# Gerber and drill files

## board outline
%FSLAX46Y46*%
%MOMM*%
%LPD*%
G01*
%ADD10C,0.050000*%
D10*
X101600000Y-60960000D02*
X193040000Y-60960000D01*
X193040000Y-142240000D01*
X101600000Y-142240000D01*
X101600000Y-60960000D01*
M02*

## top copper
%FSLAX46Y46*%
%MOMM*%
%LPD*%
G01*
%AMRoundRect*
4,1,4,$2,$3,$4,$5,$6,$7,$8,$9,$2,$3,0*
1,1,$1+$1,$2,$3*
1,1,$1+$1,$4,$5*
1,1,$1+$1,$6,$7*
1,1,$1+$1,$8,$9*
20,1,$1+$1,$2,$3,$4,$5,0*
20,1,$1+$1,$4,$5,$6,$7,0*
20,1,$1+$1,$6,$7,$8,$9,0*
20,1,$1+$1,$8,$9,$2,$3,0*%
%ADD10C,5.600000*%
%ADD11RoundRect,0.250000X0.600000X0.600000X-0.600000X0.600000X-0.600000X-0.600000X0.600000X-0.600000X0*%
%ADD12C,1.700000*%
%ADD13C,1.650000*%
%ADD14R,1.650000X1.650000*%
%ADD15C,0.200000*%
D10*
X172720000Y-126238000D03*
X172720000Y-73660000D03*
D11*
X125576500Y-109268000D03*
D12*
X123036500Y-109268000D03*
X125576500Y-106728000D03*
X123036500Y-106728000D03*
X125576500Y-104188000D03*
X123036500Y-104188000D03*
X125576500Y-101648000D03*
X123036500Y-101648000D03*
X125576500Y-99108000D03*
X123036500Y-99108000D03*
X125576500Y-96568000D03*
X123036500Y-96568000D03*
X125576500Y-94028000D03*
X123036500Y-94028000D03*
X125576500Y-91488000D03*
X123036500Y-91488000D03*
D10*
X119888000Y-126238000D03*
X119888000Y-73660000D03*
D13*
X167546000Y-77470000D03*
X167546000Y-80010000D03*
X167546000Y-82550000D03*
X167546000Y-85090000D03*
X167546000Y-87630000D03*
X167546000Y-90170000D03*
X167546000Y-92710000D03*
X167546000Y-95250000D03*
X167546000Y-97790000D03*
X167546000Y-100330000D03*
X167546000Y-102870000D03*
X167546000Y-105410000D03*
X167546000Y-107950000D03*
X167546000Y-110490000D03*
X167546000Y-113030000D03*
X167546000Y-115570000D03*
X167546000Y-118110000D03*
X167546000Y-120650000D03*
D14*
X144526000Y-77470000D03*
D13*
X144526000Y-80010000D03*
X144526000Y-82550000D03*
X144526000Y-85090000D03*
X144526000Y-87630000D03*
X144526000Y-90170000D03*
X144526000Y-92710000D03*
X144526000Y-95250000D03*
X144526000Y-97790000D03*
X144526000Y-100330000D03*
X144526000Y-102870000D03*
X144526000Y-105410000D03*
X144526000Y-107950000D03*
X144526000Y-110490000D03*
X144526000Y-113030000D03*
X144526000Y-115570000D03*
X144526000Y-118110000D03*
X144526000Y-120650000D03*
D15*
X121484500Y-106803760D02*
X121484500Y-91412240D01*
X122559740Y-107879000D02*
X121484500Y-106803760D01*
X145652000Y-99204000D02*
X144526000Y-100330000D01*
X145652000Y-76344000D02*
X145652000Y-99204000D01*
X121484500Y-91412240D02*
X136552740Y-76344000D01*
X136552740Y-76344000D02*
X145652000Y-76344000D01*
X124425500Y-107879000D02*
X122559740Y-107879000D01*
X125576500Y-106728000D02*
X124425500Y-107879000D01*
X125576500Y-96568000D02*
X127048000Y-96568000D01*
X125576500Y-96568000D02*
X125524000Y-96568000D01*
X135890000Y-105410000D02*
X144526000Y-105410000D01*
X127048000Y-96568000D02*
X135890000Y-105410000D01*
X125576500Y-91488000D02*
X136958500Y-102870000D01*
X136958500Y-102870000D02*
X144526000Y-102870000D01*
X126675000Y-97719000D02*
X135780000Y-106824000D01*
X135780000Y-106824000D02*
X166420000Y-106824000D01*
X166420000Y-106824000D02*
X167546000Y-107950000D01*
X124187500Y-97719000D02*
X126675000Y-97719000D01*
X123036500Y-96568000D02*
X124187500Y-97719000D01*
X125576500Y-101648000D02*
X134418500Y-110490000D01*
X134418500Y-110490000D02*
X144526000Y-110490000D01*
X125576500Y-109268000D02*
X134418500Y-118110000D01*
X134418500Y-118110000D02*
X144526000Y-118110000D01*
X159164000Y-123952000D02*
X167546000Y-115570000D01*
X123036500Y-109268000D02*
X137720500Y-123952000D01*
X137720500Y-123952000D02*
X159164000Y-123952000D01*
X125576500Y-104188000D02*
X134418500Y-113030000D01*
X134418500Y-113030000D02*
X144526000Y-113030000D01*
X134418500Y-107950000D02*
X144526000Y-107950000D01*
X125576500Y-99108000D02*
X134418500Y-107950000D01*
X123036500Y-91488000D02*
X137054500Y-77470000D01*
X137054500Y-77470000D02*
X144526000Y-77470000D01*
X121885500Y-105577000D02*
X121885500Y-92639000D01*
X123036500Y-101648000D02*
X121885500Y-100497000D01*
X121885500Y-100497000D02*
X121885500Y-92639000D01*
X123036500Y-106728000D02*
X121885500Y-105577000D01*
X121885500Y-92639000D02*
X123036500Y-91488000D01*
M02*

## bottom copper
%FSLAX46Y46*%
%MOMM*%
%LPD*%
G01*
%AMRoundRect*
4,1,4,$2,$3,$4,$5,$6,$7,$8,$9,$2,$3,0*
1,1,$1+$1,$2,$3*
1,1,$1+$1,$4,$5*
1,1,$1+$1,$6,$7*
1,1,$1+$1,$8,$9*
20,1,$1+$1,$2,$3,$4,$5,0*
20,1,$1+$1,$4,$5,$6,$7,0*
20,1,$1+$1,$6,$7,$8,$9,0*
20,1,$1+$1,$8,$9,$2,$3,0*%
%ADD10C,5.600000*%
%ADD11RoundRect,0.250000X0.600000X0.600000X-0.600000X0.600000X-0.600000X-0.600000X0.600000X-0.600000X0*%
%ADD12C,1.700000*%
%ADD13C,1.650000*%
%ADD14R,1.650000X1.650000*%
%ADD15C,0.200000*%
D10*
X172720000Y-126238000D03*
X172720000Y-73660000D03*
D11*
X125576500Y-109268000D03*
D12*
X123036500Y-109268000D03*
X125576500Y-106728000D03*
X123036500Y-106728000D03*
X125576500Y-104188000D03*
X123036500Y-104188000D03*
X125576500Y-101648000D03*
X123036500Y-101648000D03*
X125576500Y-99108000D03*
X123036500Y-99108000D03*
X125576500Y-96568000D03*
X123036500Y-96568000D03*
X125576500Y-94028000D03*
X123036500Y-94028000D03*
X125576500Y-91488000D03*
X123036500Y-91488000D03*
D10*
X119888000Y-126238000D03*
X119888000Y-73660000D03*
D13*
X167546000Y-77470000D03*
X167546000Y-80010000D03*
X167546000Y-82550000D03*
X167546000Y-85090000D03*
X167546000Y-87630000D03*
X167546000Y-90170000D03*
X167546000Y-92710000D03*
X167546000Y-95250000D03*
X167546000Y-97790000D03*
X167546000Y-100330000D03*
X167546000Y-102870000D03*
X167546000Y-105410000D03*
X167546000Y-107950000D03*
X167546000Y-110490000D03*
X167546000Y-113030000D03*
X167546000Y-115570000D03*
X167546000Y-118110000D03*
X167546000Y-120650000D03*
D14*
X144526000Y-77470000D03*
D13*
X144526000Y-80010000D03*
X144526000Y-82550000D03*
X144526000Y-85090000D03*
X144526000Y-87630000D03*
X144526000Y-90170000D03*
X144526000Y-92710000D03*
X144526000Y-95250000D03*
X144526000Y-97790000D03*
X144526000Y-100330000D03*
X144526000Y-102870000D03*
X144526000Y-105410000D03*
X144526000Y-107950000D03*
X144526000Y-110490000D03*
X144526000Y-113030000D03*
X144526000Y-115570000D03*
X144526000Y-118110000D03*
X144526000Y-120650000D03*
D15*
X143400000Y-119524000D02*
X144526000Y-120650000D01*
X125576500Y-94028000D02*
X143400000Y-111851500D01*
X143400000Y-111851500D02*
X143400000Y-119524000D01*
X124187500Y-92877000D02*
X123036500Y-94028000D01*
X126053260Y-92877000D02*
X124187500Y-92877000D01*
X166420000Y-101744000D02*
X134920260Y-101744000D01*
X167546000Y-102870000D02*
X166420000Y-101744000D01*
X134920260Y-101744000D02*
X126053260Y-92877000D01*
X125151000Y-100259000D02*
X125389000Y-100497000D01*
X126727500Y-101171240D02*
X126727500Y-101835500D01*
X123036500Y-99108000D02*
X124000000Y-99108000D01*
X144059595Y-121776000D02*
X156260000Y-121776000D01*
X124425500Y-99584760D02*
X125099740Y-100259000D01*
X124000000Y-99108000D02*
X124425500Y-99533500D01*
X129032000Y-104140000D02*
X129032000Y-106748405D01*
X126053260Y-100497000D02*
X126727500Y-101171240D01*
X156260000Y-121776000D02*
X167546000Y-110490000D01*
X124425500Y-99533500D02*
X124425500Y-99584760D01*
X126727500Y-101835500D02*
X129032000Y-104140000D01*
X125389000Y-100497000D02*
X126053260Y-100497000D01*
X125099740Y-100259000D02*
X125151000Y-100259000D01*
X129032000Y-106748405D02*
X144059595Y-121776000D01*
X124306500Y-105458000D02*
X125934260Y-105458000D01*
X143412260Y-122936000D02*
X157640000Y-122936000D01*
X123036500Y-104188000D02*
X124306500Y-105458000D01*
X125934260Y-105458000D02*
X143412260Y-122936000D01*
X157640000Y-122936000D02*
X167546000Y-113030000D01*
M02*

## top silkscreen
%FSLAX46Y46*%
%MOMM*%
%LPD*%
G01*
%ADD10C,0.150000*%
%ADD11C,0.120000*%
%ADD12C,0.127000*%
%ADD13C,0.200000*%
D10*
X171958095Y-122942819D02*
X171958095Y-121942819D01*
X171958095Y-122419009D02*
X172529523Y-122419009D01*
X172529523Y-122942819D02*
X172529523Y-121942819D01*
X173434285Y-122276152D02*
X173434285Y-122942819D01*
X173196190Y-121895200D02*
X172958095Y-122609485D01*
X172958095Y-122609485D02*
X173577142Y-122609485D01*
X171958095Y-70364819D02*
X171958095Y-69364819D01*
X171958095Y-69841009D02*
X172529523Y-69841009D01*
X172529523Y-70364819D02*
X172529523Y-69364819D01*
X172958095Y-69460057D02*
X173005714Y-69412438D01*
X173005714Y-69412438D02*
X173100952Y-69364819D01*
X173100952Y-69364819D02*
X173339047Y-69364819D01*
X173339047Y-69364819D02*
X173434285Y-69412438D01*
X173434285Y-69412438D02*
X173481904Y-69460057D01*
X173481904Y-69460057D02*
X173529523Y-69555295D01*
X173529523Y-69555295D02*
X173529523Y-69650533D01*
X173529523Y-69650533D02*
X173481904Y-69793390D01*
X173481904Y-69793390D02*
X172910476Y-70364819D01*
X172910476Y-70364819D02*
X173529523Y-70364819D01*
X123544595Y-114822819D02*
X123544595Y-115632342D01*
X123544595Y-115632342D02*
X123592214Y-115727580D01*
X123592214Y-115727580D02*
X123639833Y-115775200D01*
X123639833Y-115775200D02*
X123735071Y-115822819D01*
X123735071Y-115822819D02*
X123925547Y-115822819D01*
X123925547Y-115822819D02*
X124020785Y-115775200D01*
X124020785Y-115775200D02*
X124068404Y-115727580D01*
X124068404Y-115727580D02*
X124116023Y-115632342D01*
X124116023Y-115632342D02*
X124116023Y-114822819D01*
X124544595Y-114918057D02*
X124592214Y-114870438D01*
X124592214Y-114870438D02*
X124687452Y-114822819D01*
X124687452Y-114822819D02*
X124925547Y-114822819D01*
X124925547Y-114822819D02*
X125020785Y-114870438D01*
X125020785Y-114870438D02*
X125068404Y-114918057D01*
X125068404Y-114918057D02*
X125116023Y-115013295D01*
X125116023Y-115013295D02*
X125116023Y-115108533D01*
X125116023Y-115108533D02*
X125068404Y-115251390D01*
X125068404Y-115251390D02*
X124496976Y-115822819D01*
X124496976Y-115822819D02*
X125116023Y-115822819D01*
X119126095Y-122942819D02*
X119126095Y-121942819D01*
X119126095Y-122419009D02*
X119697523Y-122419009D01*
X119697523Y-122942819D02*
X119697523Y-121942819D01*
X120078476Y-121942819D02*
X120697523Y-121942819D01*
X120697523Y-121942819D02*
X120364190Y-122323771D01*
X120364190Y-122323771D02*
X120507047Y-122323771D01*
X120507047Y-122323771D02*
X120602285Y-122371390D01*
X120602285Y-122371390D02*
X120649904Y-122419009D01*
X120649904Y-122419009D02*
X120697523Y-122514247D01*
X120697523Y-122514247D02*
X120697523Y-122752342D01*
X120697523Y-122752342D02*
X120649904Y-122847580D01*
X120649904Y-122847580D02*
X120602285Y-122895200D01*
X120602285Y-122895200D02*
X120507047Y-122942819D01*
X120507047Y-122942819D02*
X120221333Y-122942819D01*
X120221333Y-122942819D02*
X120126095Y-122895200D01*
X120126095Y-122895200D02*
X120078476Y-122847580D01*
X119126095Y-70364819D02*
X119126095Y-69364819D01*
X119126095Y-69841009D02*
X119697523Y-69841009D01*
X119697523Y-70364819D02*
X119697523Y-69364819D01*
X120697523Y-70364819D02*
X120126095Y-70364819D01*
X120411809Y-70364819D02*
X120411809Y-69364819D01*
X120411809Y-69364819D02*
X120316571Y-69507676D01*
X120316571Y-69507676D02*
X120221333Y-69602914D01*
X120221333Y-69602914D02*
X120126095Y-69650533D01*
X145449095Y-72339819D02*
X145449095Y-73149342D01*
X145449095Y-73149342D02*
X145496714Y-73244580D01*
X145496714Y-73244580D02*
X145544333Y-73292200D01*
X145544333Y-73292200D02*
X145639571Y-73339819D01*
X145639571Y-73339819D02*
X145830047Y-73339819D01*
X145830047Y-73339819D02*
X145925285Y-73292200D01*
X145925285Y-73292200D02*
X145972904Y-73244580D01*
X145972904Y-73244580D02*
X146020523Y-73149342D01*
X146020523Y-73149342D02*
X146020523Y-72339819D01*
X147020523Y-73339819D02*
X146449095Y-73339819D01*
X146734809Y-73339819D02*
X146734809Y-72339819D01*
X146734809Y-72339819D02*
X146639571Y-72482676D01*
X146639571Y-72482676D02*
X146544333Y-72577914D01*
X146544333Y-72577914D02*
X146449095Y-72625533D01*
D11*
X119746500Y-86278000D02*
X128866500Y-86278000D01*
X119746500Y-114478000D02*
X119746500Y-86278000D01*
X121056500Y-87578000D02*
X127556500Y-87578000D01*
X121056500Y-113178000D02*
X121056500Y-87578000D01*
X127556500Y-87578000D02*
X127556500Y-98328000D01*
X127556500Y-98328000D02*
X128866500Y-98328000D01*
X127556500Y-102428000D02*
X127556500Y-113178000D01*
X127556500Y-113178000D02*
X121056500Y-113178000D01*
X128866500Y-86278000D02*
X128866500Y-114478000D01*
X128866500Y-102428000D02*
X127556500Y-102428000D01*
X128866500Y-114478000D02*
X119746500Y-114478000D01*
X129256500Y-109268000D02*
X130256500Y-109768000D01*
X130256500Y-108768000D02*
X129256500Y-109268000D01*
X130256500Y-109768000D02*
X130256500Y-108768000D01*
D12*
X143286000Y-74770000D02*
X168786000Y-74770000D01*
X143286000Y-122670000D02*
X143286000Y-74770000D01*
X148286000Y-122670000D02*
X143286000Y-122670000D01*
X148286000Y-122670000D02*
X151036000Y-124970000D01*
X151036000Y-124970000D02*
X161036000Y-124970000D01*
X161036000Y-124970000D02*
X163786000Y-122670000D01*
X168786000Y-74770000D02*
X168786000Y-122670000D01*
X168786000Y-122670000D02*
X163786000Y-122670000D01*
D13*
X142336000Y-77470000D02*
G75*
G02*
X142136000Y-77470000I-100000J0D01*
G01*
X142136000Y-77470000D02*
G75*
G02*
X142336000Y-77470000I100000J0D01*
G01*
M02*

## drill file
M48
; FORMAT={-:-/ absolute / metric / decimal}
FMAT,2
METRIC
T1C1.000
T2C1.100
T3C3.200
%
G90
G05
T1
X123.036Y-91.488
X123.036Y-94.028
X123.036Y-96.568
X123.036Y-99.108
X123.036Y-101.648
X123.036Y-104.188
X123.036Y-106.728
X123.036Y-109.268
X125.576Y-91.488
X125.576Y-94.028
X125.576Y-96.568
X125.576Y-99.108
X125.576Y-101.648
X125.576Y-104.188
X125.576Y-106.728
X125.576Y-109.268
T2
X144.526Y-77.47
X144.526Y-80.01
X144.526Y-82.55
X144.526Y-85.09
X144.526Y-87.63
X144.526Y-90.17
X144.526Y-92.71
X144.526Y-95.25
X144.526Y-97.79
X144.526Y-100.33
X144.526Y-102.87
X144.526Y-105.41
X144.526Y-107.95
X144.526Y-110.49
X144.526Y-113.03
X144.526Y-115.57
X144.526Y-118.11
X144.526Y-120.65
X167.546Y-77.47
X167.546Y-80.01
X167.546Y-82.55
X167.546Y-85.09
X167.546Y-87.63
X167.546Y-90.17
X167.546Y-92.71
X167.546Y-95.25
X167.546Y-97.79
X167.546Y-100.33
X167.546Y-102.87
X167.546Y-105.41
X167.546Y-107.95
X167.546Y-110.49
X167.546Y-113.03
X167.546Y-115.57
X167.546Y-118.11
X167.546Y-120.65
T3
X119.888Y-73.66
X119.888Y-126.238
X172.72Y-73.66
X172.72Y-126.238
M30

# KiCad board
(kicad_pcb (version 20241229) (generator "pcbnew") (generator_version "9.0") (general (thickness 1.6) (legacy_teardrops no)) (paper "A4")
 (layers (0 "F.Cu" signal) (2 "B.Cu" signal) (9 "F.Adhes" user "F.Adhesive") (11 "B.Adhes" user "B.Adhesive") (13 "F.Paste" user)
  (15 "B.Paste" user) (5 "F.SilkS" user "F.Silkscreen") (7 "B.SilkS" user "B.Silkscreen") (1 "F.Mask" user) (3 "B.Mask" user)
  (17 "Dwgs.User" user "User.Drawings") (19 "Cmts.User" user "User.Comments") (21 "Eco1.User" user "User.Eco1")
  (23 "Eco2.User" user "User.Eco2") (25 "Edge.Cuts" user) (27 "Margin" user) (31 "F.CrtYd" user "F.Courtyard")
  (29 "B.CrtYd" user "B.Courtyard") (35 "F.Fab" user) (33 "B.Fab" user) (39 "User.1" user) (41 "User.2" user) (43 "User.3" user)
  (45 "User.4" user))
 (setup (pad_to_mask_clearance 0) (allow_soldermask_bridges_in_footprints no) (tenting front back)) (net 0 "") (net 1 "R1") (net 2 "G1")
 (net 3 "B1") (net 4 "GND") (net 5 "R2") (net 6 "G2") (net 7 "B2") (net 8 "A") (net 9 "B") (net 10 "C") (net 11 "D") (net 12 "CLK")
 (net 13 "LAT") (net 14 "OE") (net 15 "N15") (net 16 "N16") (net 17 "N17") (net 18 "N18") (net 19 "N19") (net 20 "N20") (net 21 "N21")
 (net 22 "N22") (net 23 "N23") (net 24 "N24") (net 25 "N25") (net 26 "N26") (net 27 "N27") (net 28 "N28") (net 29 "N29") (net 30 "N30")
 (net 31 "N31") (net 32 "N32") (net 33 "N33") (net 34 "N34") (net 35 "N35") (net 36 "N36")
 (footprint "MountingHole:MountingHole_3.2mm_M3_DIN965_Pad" (layer "F.Cu") (at 172.72 126.238)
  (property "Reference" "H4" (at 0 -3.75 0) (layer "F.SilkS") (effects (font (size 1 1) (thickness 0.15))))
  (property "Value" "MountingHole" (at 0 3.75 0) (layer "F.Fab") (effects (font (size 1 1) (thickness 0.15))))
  (pad "1" thru_hole circle (at 0 0) (size 5.6 5.6) (drill 3.2) (layers "*.Cu" "*.Mask") (remove_unused_layers no) (zone_connect 2)))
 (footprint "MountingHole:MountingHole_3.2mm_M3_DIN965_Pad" (layer "F.Cu") (at 172.72 73.66)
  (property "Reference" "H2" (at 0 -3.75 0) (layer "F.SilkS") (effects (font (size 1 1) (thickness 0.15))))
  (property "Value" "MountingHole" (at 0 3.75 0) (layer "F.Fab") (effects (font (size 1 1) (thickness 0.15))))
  (pad "1" thru_hole circle (at 0 0) (size 5.6 5.6) (drill 3.2) (layers "*.Cu" "*.Mask") (remove_unused_layers no) (zone_connect 2)))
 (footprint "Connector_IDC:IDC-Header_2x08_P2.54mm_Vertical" (layer "F.Cu") (at 125.5765 109.268 180)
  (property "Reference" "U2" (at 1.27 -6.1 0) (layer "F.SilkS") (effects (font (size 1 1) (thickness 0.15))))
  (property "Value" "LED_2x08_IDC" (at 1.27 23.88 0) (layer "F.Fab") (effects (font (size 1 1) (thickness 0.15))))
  (fp_line (start 5.83 22.99) (end -3.29 22.99) (stroke (width 0.12) (type solid)) (layer "F.SilkS"))
  (fp_line (start 5.83 -5.21) (end 5.83 22.99) (stroke (width 0.12) (type solid)) (layer "F.SilkS"))
  (fp_line (start 4.52 21.69) (end -1.98 21.69) (stroke (width 0.12) (type solid)) (layer "F.SilkS"))
  (fp_line (start 4.52 -3.91) (end 4.52 21.69) (stroke (width 0.12) (type solid)) (layer "F.SilkS"))
  (fp_line (start -1.98 21.69) (end -1.98 10.94) (stroke (width 0.12) (type solid)) (layer "F.SilkS"))
  (fp_line (start -1.98 10.94) (end -3.29 10.94) (stroke (width 0.12) (type solid)) (layer "F.SilkS"))
  (fp_line (start -1.98 6.84) (end -1.98 -3.91) (stroke (width 0.12) (type solid)) (layer "F.SilkS"))
  (fp_line (start -1.98 -3.91) (end 4.52 -3.91) (stroke (width 0.12) (type solid)) (layer "F.SilkS"))
  (fp_line (start -3.29 22.99) (end -3.29 -5.21) (stroke (width 0.12) (type solid)) (layer "F.SilkS"))
  (fp_line (start -3.29 6.84) (end -1.98 6.84) (stroke (width 0.12) (type solid)) (layer "F.SilkS"))
  (fp_line (start -3.29 -5.21) (end 5.83 -5.21) (stroke (width 0.12) (type solid)) (layer "F.SilkS"))
  (fp_line (start -3.68 0) (end -4.68 -0.5) (stroke (width 0.12) (type solid)) (layer "F.SilkS"))
  (fp_line (start -4.68 0.5) (end -3.68 0) (stroke (width 0.12) (type solid)) (layer "F.SilkS"))
  (fp_line (start -4.68 -0.5) (end -4.68 0.5) (stroke (width 0.12) (type solid)) (layer "F.SilkS"))
  (pad "1" thru_hole roundrect (at 0 0 180) (size 1.7 1.7) (drill 1) (layers "*.Cu" "*.Mask") (remove_unused_layers no)
   (roundrect_rratio 0.147059) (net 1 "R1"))
  (pad "2" thru_hole circle (at 2.54 0 180) (size 1.7 1.7) (drill 1) (layers "*.Cu" "*.Mask") (remove_unused_layers no) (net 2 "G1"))
  (pad "3" thru_hole circle (at 0 2.54 180) (size 1.7 1.7) (drill 1) (layers "*.Cu" "*.Mask") (remove_unused_layers no) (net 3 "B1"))
  (pad "4" thru_hole circle (at 2.54 2.54 180) (size 1.7 1.7) (drill 1) (layers "*.Cu" "*.Mask") (remove_unused_layers no) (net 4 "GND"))
  (pad "5" thru_hole circle (at 0 5.08 180) (size 1.7 1.7) (drill 1) (layers "*.Cu" "*.Mask") (remove_unused_layers no) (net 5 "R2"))
  (pad "6" thru_hole circle (at 2.54 5.08 180) (size 1.7 1.7) (drill 1) (layers "*.Cu" "*.Mask") (remove_unused_layers no) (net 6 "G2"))
  (pad "7" thru_hole circle (at 0 7.62 180) (size 1.7 1.7) (drill 1) (layers "*.Cu" "*.Mask") (remove_unused_layers no) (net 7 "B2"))
  (pad "8" thru_hole circle (at 2.54 7.62 180) (size 1.7 1.7) (drill 1) (layers "*.Cu" "*.Mask") (remove_unused_layers no) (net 4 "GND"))
  (pad "9" thru_hole circle (at 0 10.16 180) (size 1.7 1.7) (drill 1) (layers "*.Cu" "*.Mask") (remove_unused_layers no) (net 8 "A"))
  (pad "10" thru_hole circle (at 2.54 10.16 180) (size 1.7 1.7) (drill 1) (layers "*.Cu" "*.Mask") (remove_unused_layers no) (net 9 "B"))
  (pad "11" thru_hole circle (at 0 12.7 180) (size 1.7 1.7) (drill 1) (layers "*.Cu" "*.Mask") (remove_unused_layers no) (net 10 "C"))
  (pad "12" thru_hole circle (at 2.54 12.7 180) (size 1.7 1.7) (drill 1) (layers "*.Cu" "*.Mask") (remove_unused_layers no) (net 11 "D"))
  (pad "13" thru_hole circle (at 0 15.24 180) (size 1.7 1.7) (drill 1) (layers "*.Cu" "*.Mask") (remove_unused_layers no) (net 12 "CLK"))
  (pad "14" thru_hole circle (at 2.54 15.24 180) (size 1.7 1.7) (drill 1) (layers "*.Cu" "*.Mask") (remove_unused_layers no) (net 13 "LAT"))
  (pad "15" thru_hole circle (at 0 17.78 180) (size 1.7 1.7) (drill 1) (layers "*.Cu" "*.Mask") (remove_unused_layers no) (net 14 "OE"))
  (pad "16" thru_hole circle (at 2.54 17.78 180) (size 1.7 1.7) (drill 1) (layers "*.Cu" "*.Mask") (remove_unused_layers no) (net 4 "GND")))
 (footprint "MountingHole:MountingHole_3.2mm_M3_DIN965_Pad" (layer "F.Cu") (at 119.888 126.238)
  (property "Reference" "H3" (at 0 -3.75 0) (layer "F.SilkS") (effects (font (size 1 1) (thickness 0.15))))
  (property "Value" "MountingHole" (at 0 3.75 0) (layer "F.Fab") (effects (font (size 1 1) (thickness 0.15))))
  (pad "1" thru_hole circle (at 0 0) (size 5.6 5.6) (drill 3.2) (layers "*.Cu" "*.Mask") (remove_unused_layers no) (zone_connect 2)))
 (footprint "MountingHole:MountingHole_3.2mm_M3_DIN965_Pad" (layer "F.Cu") (at 119.888 73.66)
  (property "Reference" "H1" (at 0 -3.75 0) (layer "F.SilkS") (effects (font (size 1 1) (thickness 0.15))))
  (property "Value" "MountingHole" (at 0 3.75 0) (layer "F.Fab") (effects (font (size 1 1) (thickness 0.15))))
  (pad "1" thru_hole circle (at 0 0) (size 5.6 5.6) (drill 3.2) (layers "*.Cu" "*.Mask") (remove_unused_layers no) (zone_connect 2)))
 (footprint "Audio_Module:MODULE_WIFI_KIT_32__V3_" (layer "F.Cu") (at 156.036 99.87)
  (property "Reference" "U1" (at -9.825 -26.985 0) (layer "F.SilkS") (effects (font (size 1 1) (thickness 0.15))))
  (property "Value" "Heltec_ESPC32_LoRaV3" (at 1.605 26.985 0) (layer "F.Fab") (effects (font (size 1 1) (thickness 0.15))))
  (fp_line (start -12.75 -25.1) (end 12.75 -25.1) (stroke (width 0.127) (type solid)) (layer "F.SilkS"))
  (fp_line (start -12.75 22.8) (end -12.75 -25.1) (stroke (width 0.127) (type solid)) (layer "F.SilkS"))
  (fp_line (start -7.75 22.8) (end -12.75 22.8) (stroke (width 0.127) (type solid)) (layer "F.SilkS"))
  (fp_line (start -7.75 22.8) (end -5 25.1) (stroke (width 0.127) (type solid)) (layer "F.SilkS"))
  (fp_line (start -5 25.1) (end 5 25.1) (stroke (width 0.127) (type solid)) (layer "F.SilkS"))
  (fp_line (start 5 25.1) (end 7.75 22.8) (stroke (width 0.127) (type solid)) (layer "F.SilkS"))
  (fp_line (start 12.75 -25.1) (end 12.75 22.8) (stroke (width 0.127) (type solid)) (layer "F.SilkS"))
  (fp_line (start 12.75 22.8) (end 7.75 22.8) (stroke (width 0.127) (type solid)) (layer "F.SilkS"))
  (fp_circle (center -13.8 -22.4) (end -13.7 -22.4) (stroke (width 0.2) (type solid)) (fill no) (layer "F.SilkS"))
  (pad "1" thru_hole circle (at 11.51 -22.4) (size 1.65 1.65) (drill 1.1) (layers "*.Cu" "*.Mask") (remove_unused_layers no) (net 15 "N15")
   (solder_mask_margin 0.102))
  (pad "2" thru_hole circle (at 11.51 -19.86) (size 1.65 1.65) (drill 1.1) (layers "*.Cu" "*.Mask") (remove_unused_layers no) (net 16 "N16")
   (solder_mask_margin 0.102))
  (pad "3" thru_hole circle (at 11.51 -17.32) (size 1.65 1.65) (drill 1.1) (layers "*.Cu" "*.Mask") (remove_unused_layers no) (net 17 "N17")
   (solder_mask_margin 0.102))
  (pad "4" thru_hole circle (at 11.51 -14.78) (size 1.65 1.65) (drill 1.1) (layers "*.Cu" "*.Mask") (remove_unused_layers no) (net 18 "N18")
   (solder_mask_margin 0.102))
  (pad "5" thru_hole circle (at 11.51 -12.24) (size 1.65 1.65) (drill 1.1) (layers "*.Cu" "*.Mask") (remove_unused_layers no) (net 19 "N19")
   (solder_mask_margin 0.102))
  (pad "6" thru_hole circle (at 11.51 -9.7) (size 1.65 1.65) (drill 1.1) (layers "*.Cu" "*.Mask") (remove_unused_layers no) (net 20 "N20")
   (solder_mask_margin 0.102))
  (pad "7" thru_hole circle (at 11.51 -7.16) (size 1.65 1.65) (drill 1.1) (layers "*.Cu" "*.Mask") (remove_unused_layers no) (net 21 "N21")
   (solder_mask_margin 0.102))
  (pad "8" thru_hole circle (at 11.51 -4.62) (size 1.65 1.65) (drill 1.1) (layers "*.Cu" "*.Mask") (remove_unused_layers no) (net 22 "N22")
   (solder_mask_margin 0.102))
  (pad "9" thru_hole circle (at 11.51 -2.08) (size 1.65 1.65) (drill 1.1) (layers "*.Cu" "*.Mask") (remove_unused_layers no) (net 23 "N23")
   (solder_mask_margin 0.102))
  (pad "10" thru_hole circle (at 11.51 0.46) (size 1.65 1.65) (drill 1.1) (layers "*.Cu" "*.Mask") (remove_unused_layers no) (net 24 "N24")
   (solder_mask_margin 0.102))
  (pad "11" thru_hole circle (at 11.51 3) (size 1.65 1.65) (drill 1.1) (layers "*.Cu" "*.Mask") (remove_unused_layers no) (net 13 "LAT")
   (solder_mask_margin 0.102))
  (pad "12" thru_hole circle (at 11.51 5.54) (size 1.65 1.65) (drill 1.1) (layers "*.Cu" "*.Mask") (remove_unused_layers no) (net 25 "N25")
   (solder_mask_margin 0.102))
  (pad "13" thru_hole circle (at 11.51 8.08) (size 1.65 1.65) (drill 1.1) (layers "*.Cu" "*.Mask") (remove_unused_layers no) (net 11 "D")
   (solder_mask_margin 0.102))
  (pad "14" thru_hole circle (at 11.51 10.62) (size 1.65 1.65) (drill 1.1) (layers "*.Cu" "*.Mask") (remove_unused_layers no) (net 9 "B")
   (solder_mask_margin 0.102))
  (pad "15" thru_hole circle (at 11.51 13.16) (size 1.65 1.65) (drill 1.1) (layers "*.Cu" "*.Mask") (remove_unused_layers no) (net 6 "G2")
   (solder_mask_margin 0.102))
  (pad "16" thru_hole circle (at 11.51 15.7) (size 1.65 1.65) (drill 1.1) (layers "*.Cu" "*.Mask") (remove_unused_layers no) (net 2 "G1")
   (solder_mask_margin 0.102))
  (pad "17" thru_hole circle (at 11.51 18.24) (size 1.65 1.65) (drill 1.1) (layers "*.Cu" "*.Mask") (remove_unused_layers no) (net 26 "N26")
   (solder_mask_margin 0.102))
  (pad "18" thru_hole circle (at 11.51 20.78) (size 1.65 1.65) (drill 1.1) (layers "*.Cu" "*.Mask") (remove_unused_layers no) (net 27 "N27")
   (solder_mask_margin 0.102))
  (pad "19" thru_hole rect (at -11.51 -22.4) (size 1.65 1.65) (drill 1.1) (layers "*.Cu" "*.Mask") (remove_unused_layers no) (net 4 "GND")
   (solder_mask_margin 0.102))
  (pad "20" thru_hole circle (at -11.51 -19.86) (size 1.65 1.65) (drill 1.1) (layers "*.Cu" "*.Mask") (remove_unused_layers no)
   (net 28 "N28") (solder_mask_margin 0.102))
  (pad "21" thru_hole circle (at -11.51 -17.32) (size 1.65 1.65) (drill 1.1) (layers "*.Cu" "*.Mask") (remove_unused_layers no)
   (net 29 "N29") (solder_mask_margin 0.102))
  (pad "22" thru_hole circle (at -11.51 -14.78) (size 1.65 1.65) (drill 1.1) (layers "*.Cu" "*.Mask") (remove_unused_layers no)
   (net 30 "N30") (solder_mask_margin 0.102))
  (pad "23" thru_hole circle (at -11.51 -12.24) (size 1.65 1.65) (drill 1.1) (layers "*.Cu" "*.Mask") (remove_unused_layers no)
   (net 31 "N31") (solder_mask_margin 0.102))
  (pad "24" thru_hole circle (at -11.51 -9.7) (size 1.65 1.65) (drill 1.1) (layers "*.Cu" "*.Mask") (remove_unused_layers no) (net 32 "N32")
   (solder_mask_margin 0.102))
  (pad "25" thru_hole circle (at -11.51 -7.16) (size 1.65 1.65) (drill 1.1) (layers "*.Cu" "*.Mask") (remove_unused_layers no)
   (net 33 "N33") (solder_mask_margin 0.102))
  (pad "26" thru_hole circle (at -11.51 -4.62) (size 1.65 1.65) (drill 1.1) (layers "*.Cu" "*.Mask") (remove_unused_layers no)
   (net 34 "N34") (solder_mask_margin 0.102))
  (pad "27" thru_hole circle (at -11.51 -2.08) (size 1.65 1.65) (drill 1.1) (layers "*.Cu" "*.Mask") (remove_unused_layers no)
   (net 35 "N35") (solder_mask_margin 0.102))
  (pad "28" thru_hole circle (at -11.51 0.46) (size 1.65 1.65) (drill 1.1) (layers "*.Cu" "*.Mask") (remove_unused_layers no) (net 3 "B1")
   (solder_mask_margin 0.102))
  (pad "29" thru_hole circle (at -11.51 3) (size 1.65 1.65) (drill 1.1) (layers "*.Cu" "*.Mask") (remove_unused_layers no) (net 14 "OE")
   (solder_mask_margin 0.102))
  (pad "30" thru_hole circle (at -11.51 5.54) (size 1.65 1.65) (drill 1.1) (layers "*.Cu" "*.Mask") (remove_unused_layers no) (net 10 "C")
   (solder_mask_margin 0.102))
  (pad "31" thru_hole circle (at -11.51 8.08) (size 1.65 1.65) (drill 1.1) (layers "*.Cu" "*.Mask") (remove_unused_layers no) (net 8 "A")
   (solder_mask_margin 0.102))
  (pad "32" thru_hole circle (at -11.51 10.62) (size 1.65 1.65) (drill 1.1) (layers "*.Cu" "*.Mask") (remove_unused_layers no) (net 7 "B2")
   (solder_mask_margin 0.102))
  (pad "33" thru_hole circle (at -11.51 13.16) (size 1.65 1.65) (drill 1.1) (layers "*.Cu" "*.Mask") (remove_unused_layers no) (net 5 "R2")
   (solder_mask_margin 0.102))
  (pad "34" thru_hole circle (at -11.51 15.7) (size 1.65 1.65) (drill 1.1) (layers "*.Cu" "*.Mask") (remove_unused_layers no) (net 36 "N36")
   (solder_mask_margin 0.102))
  (pad "35" thru_hole circle (at -11.51 18.24) (size 1.65 1.65) (drill 1.1) (layers "*.Cu" "*.Mask") (remove_unused_layers no) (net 1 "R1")
   (solder_mask_margin 0.102))
  (pad "36" thru_hole circle (at -11.51 20.78) (size 1.65 1.65) (drill 1.1) (layers "*.Cu" "*.Mask") (remove_unused_layers no)
   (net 12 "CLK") (solder_mask_margin 0.102)))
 (gr_rect (start 101.6 60.96) (end 193.04 142.24) (stroke (width 0.05) (type default)) (fill no) (layer "Edge.Cuts"))
 (segment (start 121.4845 106.80376) (end 121.4845 91.41224) (width 0.2) (layer "F.Cu") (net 3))
 (segment (start 122.55974 107.879) (end 121.4845 106.80376) (width 0.2) (layer "F.Cu") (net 3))
 (segment (start 145.652 99.204) (end 144.526 100.33) (width 0.2) (layer "F.Cu") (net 3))
 (segment (start 145.652 76.344) (end 145.652 99.204) (width 0.2) (layer "F.Cu") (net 3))
 (segment (start 121.4845 91.41224) (end 136.55274 76.344) (width 0.2) (layer "F.Cu") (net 3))
 (segment (start 136.55274 76.344) (end 145.652 76.344) (width 0.2) (layer "F.Cu") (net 3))
 (segment (start 124.4255 107.879) (end 122.55974 107.879) (width 0.2) (layer "F.Cu") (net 3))
 (segment (start 125.5765 106.728) (end 124.4255 107.879) (width 0.2) (layer "F.Cu") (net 3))
 (segment (start 125.5765 96.568) (end 127.048 96.568) (width 0.2) (layer "F.Cu") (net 10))
 (segment (start 125.5765 96.568) (end 125.524 96.568) (width 0.2) (layer "F.Cu") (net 10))
 (segment (start 135.89 105.41) (end 144.526 105.41) (width 0.2) (layer "F.Cu") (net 10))
 (segment (start 127.048 96.568) (end 135.89 105.41) (width 0.2) (layer "F.Cu") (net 10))
 (segment (start 125.5765 91.488) (end 136.9585 102.87) (width 0.2) (layer "F.Cu") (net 14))
 (segment (start 136.9585 102.87) (end 144.526 102.87) (width 0.2) (layer "F.Cu") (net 14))
 (segment (start 143.4 119.524) (end 144.526 120.65) (width 0.2) (layer "B.Cu") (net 12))
 (segment (start 125.5765 94.028) (end 143.4 111.8515) (width 0.2) (layer "B.Cu") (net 12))
 (segment (start 143.4 111.8515) (end 143.4 119.524) (width 0.2) (layer "B.Cu") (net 12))
 (segment (start 126.675 97.719) (end 135.78 106.824) (width 0.2) (layer "F.Cu") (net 11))
 (segment (start 135.78 106.824) (end 166.42 106.824) (width 0.2) (layer "F.Cu") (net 11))
 (segment (start 166.42 106.824) (end 167.546 107.95) (width 0.2) (layer "F.Cu") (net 11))
 (segment (start 124.1875 97.719) (end 126.675 97.719) (width 0.2) (layer "F.Cu") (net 11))
 (segment (start 123.0365 96.568) (end 124.1875 97.719) (width 0.2) (layer "F.Cu") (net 11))
 (segment (start 125.5765 101.648) (end 134.4185 110.49) (width 0.2) (layer "F.Cu") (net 7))
 (segment (start 134.4185 110.49) (end 144.526 110.49) (width 0.2) (layer "F.Cu") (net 7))
 (segment (start 124.1875 92.877) (end 123.0365 94.028) (width 0.2) (layer "B.Cu") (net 13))
 (segment (start 126.05326 92.877) (end 124.1875 92.877) (width 0.2) (layer "B.Cu") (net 13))
 (segment (start 166.42 101.744) (end 134.92026 101.744) (width 0.2) (layer "B.Cu") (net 13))
 (segment (start 167.546 102.87) (end 166.42 101.744) (width 0.2) (layer "B.Cu") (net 13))
 (segment (start 134.92026 101.744) (end 126.05326 92.877) (width 0.2) (layer "B.Cu") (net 13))
 (segment (start 125.5765 109.268) (end 134.4185 118.11) (width 0.2) (layer "F.Cu") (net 1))
 (segment (start 134.4185 118.11) (end 144.526 118.11) (width 0.2) (layer "F.Cu") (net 1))
 (segment (start 159.164 123.952) (end 167.546 115.57) (width 0.2) (layer "F.Cu") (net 2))
 (segment (start 123.0365 109.268) (end 137.7205 123.952) (width 0.2) (layer "F.Cu") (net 2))
 (segment (start 137.7205 123.952) (end 159.164 123.952) (width 0.2) (layer "F.Cu") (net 2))
 (segment (start 125.5765 104.188) (end 134.4185 113.03) (width 0.2) (layer "F.Cu") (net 5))
 (segment (start 134.4185 113.03) (end 144.526 113.03) (width 0.2) (layer "F.Cu") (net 5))
 (segment (start 125.151 100.259) (end 125.389 100.497) (width 0.2) (layer "B.Cu") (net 9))
 (segment (start 126.7275 101.17124) (end 126.7275 101.8355) (width 0.2) (layer "B.Cu") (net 9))
 (segment (start 123.0365 99.108) (end 124 99.108) (width 0.2) (layer "B.Cu") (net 9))
 (segment (start 144.059595 121.776) (end 156.26 121.776) (width 0.2) (layer "B.Cu") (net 9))
 (segment (start 124.4255 99.58476) (end 125.09974 100.259) (width 0.2) (layer "B.Cu") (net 9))
 (segment (start 124 99.108) (end 124.4255 99.5335) (width 0.2) (layer "B.Cu") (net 9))
 (segment (start 129.032 104.14) (end 129.032 106.748405) (width 0.2) (layer "B.Cu") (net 9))
 (segment (start 126.05326 100.497) (end 126.7275 101.17124) (width 0.2) (layer "B.Cu") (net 9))
 (segment (start 156.26 121.776) (end 167.546 110.49) (width 0.2) (layer "B.Cu") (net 9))
 (segment (start 124.4255 99.5335) (end 124.4255 99.58476) (width 0.2) (layer "B.Cu") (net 9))
 (segment (start 126.7275 101.8355) (end 129.032 104.14) (width 0.2) (layer "B.Cu") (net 9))
 (segment (start 125.389 100.497) (end 126.05326 100.497) (width 0.2) (layer "B.Cu") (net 9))
 (segment (start 125.09974 100.259) (end 125.151 100.259) (width 0.2) (layer "B.Cu") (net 9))
 (segment (start 129.032 106.748405) (end 144.059595 121.776) (width 0.2) (layer "B.Cu") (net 9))
 (segment (start 134.4185 107.95) (end 144.526 107.95) (width 0.2) (layer "F.Cu") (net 8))
 (segment (start 125.5765 99.108) (end 134.4185 107.95) (width 0.2) (layer "F.Cu") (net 8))
 (segment (start 124.3065 105.458) (end 125.93426 105.458) (width 0.2) (layer "B.Cu") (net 6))
 (segment (start 143.41226 122.936) (end 157.64 122.936) (width 0.2) (layer "B.Cu") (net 6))
 (segment (start 123.0365 104.188) (end 124.3065 105.458) (width 0.2) (layer "B.Cu") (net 6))
 (segment (start 125.93426 105.458) (end 143.41226 122.936) (width 0.2) (layer "B.Cu") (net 6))
 (segment (start 157.64 122.936) (end 167.546 113.03) (width 0.2) (layer "B.Cu") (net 6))
 (segment (start 123.0365 91.488) (end 137.0545 77.47) (width 0.2) (layer "F.Cu") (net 4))
 (segment (start 137.0545 77.47) (end 144.526 77.47) (width 0.2) (layer "F.Cu") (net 4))
 (segment (start 121.8855 105.577) (end 121.8855 92.639) (width 0.2) (layer "F.Cu") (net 4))
 (segment (start 123.0365 101.648) (end 121.8855 100.497) (width 0.2) (layer "F.Cu") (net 4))
 (segment (start 121.8855 100.497) (end 121.8855 92.639) (width 0.2) (layer "F.Cu") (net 4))
 (segment (start 123.0365 106.728) (end 121.8855 105.577) (width 0.2) (layer "F.Cu") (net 4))
 (segment (start 121.8855 92.639) (end 123.0365 91.488) (width 0.2) (layer "F.Cu") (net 4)))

